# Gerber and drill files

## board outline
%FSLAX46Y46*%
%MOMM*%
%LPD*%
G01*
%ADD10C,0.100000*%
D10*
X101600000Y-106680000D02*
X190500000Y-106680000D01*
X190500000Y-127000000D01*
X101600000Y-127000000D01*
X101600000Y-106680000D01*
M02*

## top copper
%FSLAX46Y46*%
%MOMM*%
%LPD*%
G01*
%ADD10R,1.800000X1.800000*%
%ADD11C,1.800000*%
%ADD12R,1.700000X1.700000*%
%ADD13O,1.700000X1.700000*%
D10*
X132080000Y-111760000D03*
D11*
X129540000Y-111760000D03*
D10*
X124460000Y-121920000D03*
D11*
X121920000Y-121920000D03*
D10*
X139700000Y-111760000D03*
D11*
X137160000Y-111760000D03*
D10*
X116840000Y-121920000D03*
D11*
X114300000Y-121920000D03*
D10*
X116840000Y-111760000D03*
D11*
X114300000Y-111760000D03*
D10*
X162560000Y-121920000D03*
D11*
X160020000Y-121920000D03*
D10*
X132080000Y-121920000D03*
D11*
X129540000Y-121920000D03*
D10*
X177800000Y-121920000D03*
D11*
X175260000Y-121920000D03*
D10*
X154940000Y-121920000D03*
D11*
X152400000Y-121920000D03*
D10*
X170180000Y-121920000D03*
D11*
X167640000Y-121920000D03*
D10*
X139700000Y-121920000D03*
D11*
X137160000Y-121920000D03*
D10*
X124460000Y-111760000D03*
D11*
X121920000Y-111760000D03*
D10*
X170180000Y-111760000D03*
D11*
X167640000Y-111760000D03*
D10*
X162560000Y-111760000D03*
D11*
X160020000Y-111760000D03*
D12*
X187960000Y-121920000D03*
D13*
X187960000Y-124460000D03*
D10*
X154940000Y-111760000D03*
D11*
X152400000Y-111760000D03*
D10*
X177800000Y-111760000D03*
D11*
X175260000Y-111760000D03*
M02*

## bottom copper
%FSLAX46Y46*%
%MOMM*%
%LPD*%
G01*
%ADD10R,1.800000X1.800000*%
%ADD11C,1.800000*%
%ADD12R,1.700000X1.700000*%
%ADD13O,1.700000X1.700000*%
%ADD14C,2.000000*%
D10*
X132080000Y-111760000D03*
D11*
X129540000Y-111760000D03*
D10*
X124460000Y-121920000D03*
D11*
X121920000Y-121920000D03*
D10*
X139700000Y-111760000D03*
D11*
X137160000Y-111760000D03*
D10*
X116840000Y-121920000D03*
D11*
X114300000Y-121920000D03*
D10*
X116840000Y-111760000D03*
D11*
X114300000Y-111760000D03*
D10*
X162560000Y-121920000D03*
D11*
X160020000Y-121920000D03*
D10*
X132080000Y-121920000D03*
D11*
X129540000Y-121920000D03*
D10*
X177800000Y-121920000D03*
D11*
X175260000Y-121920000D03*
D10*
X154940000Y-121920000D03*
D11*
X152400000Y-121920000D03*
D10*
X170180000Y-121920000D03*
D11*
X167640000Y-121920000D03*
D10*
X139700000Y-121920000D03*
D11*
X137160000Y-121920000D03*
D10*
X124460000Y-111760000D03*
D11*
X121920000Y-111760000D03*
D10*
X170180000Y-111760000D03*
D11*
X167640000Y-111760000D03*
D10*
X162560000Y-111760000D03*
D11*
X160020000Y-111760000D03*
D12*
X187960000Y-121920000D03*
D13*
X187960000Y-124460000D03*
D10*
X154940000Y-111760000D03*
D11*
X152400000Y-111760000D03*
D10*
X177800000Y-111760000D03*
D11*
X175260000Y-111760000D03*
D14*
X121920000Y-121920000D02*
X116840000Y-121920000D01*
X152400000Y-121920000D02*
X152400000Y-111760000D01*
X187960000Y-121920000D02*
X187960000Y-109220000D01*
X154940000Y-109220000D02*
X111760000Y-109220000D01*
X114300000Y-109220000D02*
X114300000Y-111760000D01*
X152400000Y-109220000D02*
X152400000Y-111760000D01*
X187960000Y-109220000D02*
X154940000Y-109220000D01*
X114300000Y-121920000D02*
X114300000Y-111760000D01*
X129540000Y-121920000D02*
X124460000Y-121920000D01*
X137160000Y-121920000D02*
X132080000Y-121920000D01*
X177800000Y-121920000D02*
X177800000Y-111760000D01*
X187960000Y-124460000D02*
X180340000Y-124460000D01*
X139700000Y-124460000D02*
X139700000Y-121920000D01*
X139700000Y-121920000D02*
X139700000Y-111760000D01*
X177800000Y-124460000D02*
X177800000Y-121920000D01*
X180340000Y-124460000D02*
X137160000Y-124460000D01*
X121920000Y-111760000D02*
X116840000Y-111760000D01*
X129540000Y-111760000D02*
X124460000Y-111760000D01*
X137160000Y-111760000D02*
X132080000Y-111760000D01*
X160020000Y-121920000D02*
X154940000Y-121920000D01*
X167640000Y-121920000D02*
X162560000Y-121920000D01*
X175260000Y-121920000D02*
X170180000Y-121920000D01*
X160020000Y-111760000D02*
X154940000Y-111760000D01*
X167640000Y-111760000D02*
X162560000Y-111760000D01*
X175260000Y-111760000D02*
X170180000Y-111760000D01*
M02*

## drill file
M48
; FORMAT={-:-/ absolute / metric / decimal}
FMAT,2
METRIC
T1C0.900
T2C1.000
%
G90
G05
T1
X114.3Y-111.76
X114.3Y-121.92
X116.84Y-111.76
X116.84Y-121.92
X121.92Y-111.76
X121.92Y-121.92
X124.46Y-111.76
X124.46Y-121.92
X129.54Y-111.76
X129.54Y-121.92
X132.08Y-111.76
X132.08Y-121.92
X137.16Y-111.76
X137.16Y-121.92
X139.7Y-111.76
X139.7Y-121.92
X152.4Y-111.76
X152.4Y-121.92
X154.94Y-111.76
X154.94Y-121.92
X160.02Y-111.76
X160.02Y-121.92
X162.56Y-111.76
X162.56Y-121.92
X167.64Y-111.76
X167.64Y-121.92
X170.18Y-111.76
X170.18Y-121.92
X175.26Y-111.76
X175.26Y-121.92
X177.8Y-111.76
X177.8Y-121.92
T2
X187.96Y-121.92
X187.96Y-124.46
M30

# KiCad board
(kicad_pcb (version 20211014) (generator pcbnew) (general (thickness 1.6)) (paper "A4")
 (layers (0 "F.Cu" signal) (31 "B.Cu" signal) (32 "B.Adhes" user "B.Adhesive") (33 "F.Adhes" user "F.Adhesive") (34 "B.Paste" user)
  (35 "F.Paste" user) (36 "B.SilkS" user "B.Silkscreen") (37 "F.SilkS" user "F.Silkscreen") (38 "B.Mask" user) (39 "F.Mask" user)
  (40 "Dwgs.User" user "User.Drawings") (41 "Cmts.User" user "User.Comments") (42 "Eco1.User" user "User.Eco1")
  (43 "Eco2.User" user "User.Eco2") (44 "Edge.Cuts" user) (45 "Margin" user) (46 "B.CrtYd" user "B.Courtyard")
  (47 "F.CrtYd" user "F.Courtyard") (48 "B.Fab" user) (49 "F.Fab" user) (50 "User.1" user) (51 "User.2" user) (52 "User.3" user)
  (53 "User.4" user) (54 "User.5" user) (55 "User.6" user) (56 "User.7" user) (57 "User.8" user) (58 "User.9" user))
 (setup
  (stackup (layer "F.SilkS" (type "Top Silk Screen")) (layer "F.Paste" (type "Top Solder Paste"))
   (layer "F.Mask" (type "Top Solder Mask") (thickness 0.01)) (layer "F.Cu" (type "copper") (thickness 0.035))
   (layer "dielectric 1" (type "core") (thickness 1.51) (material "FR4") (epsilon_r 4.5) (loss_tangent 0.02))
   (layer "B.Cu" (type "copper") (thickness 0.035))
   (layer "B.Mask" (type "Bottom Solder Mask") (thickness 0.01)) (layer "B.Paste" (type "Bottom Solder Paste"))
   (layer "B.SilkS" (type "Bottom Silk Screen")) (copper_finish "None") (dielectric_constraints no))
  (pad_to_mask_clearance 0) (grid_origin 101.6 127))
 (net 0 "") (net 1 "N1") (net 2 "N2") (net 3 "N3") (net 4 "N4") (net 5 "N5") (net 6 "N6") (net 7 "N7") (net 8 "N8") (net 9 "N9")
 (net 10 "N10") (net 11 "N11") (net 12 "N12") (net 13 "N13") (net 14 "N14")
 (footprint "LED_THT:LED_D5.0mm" (layer "F.Cu") (at 132.08 111.76 180)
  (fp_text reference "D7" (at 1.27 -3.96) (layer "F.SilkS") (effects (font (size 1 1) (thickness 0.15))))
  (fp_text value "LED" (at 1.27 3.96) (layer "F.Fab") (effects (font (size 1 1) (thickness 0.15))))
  (pad "1" thru_hole rect (at 0 0 180) (size 1.8 1.8) (drill 0.9) (layers *.Cu *.Mask) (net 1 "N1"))
  (pad "2" thru_hole circle (at 2.54 0 180) (size 1.8 1.8) (drill 0.9) (layers *.Cu *.Mask) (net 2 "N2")))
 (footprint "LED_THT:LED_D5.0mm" (layer "F.Cu") (at 124.46 121.92 180)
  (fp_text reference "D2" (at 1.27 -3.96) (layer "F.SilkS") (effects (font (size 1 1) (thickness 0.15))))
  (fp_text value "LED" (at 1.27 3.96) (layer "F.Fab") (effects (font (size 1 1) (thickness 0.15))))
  (pad "1" thru_hole rect (at 0 0 180) (size 1.8 1.8) (drill 0.9) (layers *.Cu *.Mask) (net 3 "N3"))
  (pad "2" thru_hole circle (at 2.54 0 180) (size 1.8 1.8) (drill 0.9) (layers *.Cu *.Mask) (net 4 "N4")))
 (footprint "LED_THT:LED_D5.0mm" (layer "F.Cu") (at 139.7 111.76 180)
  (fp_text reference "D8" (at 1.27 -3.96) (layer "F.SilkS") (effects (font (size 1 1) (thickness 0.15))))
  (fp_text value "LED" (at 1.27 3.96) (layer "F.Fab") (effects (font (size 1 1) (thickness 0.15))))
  (pad "1" thru_hole rect (at 0 0 180) (size 1.8 1.8) (drill 0.9) (layers *.Cu *.Mask) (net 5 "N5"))
  (pad "2" thru_hole circle (at 2.54 0 180) (size 1.8 1.8) (drill 0.9) (layers *.Cu *.Mask) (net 1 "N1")))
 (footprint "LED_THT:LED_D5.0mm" (layer "F.Cu") (at 116.84 121.92 180)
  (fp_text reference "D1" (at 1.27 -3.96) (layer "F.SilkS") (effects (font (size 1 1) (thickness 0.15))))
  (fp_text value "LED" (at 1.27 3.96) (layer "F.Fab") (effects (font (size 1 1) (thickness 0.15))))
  (pad "1" thru_hole rect (at 0 0 180) (size 1.8 1.8) (drill 0.9) (layers *.Cu *.Mask) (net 4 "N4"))
  (pad "2" thru_hole circle (at 2.54 0 180) (size 1.8 1.8) (drill 0.9) (layers *.Cu *.Mask) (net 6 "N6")))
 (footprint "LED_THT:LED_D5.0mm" (layer "F.Cu") (at 116.84 111.76 180)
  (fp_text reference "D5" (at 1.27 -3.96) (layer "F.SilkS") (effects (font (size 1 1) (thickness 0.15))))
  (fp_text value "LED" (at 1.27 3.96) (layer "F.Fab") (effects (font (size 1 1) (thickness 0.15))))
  (pad "1" thru_hole rect (at 0 0 180) (size 1.8 1.8) (drill 0.9) (layers *.Cu *.Mask) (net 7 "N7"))
  (pad "2" thru_hole circle (at 2.54 0 180) (size 1.8 1.8) (drill 0.9) (layers *.Cu *.Mask) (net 6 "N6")))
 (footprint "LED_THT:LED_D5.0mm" (layer "F.Cu") (at 162.56 121.92 180)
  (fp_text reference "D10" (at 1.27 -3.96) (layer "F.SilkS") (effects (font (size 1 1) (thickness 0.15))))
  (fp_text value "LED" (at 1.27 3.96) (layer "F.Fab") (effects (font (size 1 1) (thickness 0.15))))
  (pad "1" thru_hole rect (at 0 0 180) (size 1.8 1.8) (drill 0.9) (layers *.Cu *.Mask) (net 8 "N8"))
  (pad "2" thru_hole circle (at 2.54 0 180) (size 1.8 1.8) (drill 0.9) (layers *.Cu *.Mask) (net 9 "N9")))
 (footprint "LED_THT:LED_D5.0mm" (layer "F.Cu") (at 132.08 121.92 180)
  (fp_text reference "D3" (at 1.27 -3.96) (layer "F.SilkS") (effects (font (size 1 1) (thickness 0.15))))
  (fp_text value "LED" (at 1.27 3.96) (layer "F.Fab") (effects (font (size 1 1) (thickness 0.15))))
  (pad "1" thru_hole rect (at 0 0 180) (size 1.8 1.8) (drill 0.9) (layers *.Cu *.Mask) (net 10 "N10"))
  (pad "2" thru_hole circle (at 2.54 0 180) (size 1.8 1.8) (drill 0.9) (layers *.Cu *.Mask) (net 3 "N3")))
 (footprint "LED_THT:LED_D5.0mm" (layer "F.Cu") (at 177.8 121.92 180)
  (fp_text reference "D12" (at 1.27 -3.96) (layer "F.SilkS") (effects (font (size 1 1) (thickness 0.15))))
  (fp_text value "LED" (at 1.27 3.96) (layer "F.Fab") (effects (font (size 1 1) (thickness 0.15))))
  (pad "1" thru_hole rect (at 0 0 180) (size 1.8 1.8) (drill 0.9) (layers *.Cu *.Mask) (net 5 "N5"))
  (pad "2" thru_hole circle (at 2.54 0 180) (size 1.8 1.8) (drill 0.9) (layers *.Cu *.Mask) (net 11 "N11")))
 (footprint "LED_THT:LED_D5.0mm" (layer "F.Cu") (at 154.94 121.92 180)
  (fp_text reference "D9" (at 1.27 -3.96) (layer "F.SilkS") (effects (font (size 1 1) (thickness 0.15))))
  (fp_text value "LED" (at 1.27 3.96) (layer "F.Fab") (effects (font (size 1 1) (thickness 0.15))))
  (pad "1" thru_hole rect (at 0 0 180) (size 1.8 1.8) (drill 0.9) (layers *.Cu *.Mask) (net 9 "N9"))
  (pad "2" thru_hole circle (at 2.54 0 180) (size 1.8 1.8) (drill 0.9) (layers *.Cu *.Mask) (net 6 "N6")))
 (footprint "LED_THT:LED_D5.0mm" (layer "F.Cu") (at 170.18 121.92 180)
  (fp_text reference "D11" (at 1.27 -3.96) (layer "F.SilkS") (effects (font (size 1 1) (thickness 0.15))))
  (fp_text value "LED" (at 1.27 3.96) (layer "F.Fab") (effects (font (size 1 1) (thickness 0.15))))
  (pad "1" thru_hole rect (at 0 0 180) (size 1.8 1.8) (drill 0.9) (layers *.Cu *.Mask) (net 11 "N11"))
  (pad "2" thru_hole circle (at 2.54 0 180) (size 1.8 1.8) (drill 0.9) (layers *.Cu *.Mask) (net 8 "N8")))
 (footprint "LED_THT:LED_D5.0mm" (layer "F.Cu") (at 139.7 121.92 180)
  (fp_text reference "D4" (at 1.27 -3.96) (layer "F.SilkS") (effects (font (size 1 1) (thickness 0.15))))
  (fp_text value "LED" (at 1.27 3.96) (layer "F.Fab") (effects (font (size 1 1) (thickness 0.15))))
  (pad "1" thru_hole rect (at 0 0 180) (size 1.8 1.8) (drill 0.9) (layers *.Cu *.Mask) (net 5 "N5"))
  (pad "2" thru_hole circle (at 2.54 0 180) (size 1.8 1.8) (drill 0.9) (layers *.Cu *.Mask) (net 10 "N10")))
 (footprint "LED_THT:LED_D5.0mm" (layer "F.Cu") (at 124.46 111.76 180)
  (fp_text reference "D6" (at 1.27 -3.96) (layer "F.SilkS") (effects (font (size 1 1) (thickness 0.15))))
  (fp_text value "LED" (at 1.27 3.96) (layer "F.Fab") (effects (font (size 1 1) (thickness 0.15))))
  (pad "1" thru_hole rect (at 0 0 180) (size 1.8 1.8) (drill 0.9) (layers *.Cu *.Mask) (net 2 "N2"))
  (pad "2" thru_hole circle (at 2.54 0 180) (size 1.8 1.8) (drill 0.9) (layers *.Cu *.Mask) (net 7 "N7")))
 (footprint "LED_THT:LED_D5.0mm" (layer "F.Cu") (at 170.18 111.76 180)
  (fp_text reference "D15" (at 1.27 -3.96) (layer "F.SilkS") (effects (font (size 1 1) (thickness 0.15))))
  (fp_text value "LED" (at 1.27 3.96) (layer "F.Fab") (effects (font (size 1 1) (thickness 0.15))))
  (pad "1" thru_hole rect (at 0 0 180) (size 1.8 1.8) (drill 0.9) (layers *.Cu *.Mask) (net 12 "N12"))
  (pad "2" thru_hole circle (at 2.54 0 180) (size 1.8 1.8) (drill 0.9) (layers *.Cu *.Mask) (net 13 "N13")))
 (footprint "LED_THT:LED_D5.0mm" (layer "F.Cu") (at 162.56 111.76 180)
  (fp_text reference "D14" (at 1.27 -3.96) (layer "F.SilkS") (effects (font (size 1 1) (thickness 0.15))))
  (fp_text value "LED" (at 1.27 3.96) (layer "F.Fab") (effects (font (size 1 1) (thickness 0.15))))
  (pad "1" thru_hole rect (at 0 0 180) (size 1.8 1.8) (drill 0.9) (layers *.Cu *.Mask) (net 13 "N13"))
  (pad "2" thru_hole circle (at 2.54 0 180) (size 1.8 1.8) (drill 0.9) (layers *.Cu *.Mask) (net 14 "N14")))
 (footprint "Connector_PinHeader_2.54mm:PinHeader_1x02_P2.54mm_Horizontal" (layer "F.Cu") (at 187.96 121.92)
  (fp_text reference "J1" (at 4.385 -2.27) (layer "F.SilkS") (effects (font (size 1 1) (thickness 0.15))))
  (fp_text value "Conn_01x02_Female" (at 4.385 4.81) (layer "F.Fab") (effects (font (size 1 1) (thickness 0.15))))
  (pad "1" thru_hole rect (at 0 0) (size 1.7 1.7) (drill 1) (layers *.Cu *.Mask) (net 6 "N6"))
  (pad "2" thru_hole oval (at 0 2.54) (size 1.7 1.7) (drill 1) (layers *.Cu *.Mask) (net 5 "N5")))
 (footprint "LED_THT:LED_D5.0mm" (layer "F.Cu") (at 154.94 111.76 180)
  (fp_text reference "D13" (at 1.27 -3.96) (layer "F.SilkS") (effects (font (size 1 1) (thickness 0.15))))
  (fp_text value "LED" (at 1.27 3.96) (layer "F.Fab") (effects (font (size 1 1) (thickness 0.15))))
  (pad "1" thru_hole rect (at 0 0 180) (size 1.8 1.8) (drill 0.9) (layers *.Cu *.Mask) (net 14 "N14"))
  (pad "2" thru_hole circle (at 2.54 0 180) (size 1.8 1.8) (drill 0.9) (layers *.Cu *.Mask) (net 6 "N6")))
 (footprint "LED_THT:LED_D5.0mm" (layer "F.Cu") (at 177.8 111.76 180)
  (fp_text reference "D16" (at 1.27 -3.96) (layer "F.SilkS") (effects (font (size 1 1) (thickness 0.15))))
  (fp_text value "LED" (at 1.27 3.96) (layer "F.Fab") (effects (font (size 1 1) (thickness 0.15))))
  (pad "1" thru_hole rect (at 0 0 180) (size 1.8 1.8) (drill 0.9) (layers *.Cu *.Mask) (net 5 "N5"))
  (pad "2" thru_hole circle (at 2.54 0 180) (size 1.8 1.8) (drill 0.9) (layers *.Cu *.Mask) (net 12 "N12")))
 (gr_rect (start 101.6 127) (end 190.5 106.68) (layer "Edge.Cuts") (width 0.1) (fill none))
 (segment (start 121.92 121.92) (end 116.84 121.92) (width 2) (layer "B.Cu") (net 4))
 (segment (start 152.4 121.92) (end 152.4 111.76) (width 2) (layer "B.Cu") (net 6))
 (segment (start 187.96 121.92) (end 187.96 109.22) (width 2) (layer "B.Cu") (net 6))
 (segment (start 154.94 109.22) (end 111.76 109.22) (width 2) (layer "B.Cu") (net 6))
 (segment (start 114.3 109.22) (end 114.3 111.76) (width 2) (layer "B.Cu") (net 6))
 (segment (start 152.4 109.22) (end 152.4 111.76) (width 2) (layer "B.Cu") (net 6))
 (segment (start 187.96 109.22) (end 154.94 109.22) (width 2) (layer "B.Cu") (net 6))
 (segment (start 114.3 121.92) (end 114.3 111.76) (width 2) (layer "B.Cu") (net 6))
 (segment (start 129.54 121.92) (end 124.46 121.92) (width 2) (layer "B.Cu") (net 3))
 (segment (start 137.16 121.92) (end 132.08 121.92) (width 2) (layer "B.Cu") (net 10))
 (segment (start 177.8 121.92) (end 177.8 111.76) (width 2) (layer "B.Cu") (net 5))
 (segment (start 187.96 124.46) (end 180.34 124.46) (width 2) (layer "B.Cu") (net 5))
 (segment (start 139.7 124.46) (end 139.7 121.92) (width 2) (layer "B.Cu") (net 5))
 (segment (start 139.7 121.92) (end 139.7 111.76) (width 2) (layer "B.Cu") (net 5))
 (segment (start 177.8 124.46) (end 177.8 121.92) (width 2) (layer "B.Cu") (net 5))
 (segment (start 180.34 124.46) (end 137.16 124.46) (width 2) (layer "B.Cu") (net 5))
 (segment (start 121.92 111.76) (end 116.84 111.76) (width 2) (layer "B.Cu") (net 7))
 (segment (start 129.54 111.76) (end 124.46 111.76) (width 2) (layer "B.Cu") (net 2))
 (segment (start 137.16 111.76) (end 132.08 111.76) (width 2) (layer "B.Cu") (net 1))
 (segment (start 160.02 121.92) (end 154.94 121.92) (width 2) (layer "B.Cu") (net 9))
 (segment (start 167.64 121.92) (end 162.56 121.92) (width 2) (layer "B.Cu") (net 8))
 (segment (start 175.26 121.92) (end 170.18 121.92) (width 2) (layer "B.Cu") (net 11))
 (segment (start 160.02 111.76) (end 154.94 111.76) (width 2) (layer "B.Cu") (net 14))
 (segment (start 167.64 111.76) (end 162.56 111.76) (width 2) (layer "B.Cu") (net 13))
 (segment (start 175.26 111.76) (end 170.18 111.76) (width 2) (layer "B.Cu") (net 12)))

